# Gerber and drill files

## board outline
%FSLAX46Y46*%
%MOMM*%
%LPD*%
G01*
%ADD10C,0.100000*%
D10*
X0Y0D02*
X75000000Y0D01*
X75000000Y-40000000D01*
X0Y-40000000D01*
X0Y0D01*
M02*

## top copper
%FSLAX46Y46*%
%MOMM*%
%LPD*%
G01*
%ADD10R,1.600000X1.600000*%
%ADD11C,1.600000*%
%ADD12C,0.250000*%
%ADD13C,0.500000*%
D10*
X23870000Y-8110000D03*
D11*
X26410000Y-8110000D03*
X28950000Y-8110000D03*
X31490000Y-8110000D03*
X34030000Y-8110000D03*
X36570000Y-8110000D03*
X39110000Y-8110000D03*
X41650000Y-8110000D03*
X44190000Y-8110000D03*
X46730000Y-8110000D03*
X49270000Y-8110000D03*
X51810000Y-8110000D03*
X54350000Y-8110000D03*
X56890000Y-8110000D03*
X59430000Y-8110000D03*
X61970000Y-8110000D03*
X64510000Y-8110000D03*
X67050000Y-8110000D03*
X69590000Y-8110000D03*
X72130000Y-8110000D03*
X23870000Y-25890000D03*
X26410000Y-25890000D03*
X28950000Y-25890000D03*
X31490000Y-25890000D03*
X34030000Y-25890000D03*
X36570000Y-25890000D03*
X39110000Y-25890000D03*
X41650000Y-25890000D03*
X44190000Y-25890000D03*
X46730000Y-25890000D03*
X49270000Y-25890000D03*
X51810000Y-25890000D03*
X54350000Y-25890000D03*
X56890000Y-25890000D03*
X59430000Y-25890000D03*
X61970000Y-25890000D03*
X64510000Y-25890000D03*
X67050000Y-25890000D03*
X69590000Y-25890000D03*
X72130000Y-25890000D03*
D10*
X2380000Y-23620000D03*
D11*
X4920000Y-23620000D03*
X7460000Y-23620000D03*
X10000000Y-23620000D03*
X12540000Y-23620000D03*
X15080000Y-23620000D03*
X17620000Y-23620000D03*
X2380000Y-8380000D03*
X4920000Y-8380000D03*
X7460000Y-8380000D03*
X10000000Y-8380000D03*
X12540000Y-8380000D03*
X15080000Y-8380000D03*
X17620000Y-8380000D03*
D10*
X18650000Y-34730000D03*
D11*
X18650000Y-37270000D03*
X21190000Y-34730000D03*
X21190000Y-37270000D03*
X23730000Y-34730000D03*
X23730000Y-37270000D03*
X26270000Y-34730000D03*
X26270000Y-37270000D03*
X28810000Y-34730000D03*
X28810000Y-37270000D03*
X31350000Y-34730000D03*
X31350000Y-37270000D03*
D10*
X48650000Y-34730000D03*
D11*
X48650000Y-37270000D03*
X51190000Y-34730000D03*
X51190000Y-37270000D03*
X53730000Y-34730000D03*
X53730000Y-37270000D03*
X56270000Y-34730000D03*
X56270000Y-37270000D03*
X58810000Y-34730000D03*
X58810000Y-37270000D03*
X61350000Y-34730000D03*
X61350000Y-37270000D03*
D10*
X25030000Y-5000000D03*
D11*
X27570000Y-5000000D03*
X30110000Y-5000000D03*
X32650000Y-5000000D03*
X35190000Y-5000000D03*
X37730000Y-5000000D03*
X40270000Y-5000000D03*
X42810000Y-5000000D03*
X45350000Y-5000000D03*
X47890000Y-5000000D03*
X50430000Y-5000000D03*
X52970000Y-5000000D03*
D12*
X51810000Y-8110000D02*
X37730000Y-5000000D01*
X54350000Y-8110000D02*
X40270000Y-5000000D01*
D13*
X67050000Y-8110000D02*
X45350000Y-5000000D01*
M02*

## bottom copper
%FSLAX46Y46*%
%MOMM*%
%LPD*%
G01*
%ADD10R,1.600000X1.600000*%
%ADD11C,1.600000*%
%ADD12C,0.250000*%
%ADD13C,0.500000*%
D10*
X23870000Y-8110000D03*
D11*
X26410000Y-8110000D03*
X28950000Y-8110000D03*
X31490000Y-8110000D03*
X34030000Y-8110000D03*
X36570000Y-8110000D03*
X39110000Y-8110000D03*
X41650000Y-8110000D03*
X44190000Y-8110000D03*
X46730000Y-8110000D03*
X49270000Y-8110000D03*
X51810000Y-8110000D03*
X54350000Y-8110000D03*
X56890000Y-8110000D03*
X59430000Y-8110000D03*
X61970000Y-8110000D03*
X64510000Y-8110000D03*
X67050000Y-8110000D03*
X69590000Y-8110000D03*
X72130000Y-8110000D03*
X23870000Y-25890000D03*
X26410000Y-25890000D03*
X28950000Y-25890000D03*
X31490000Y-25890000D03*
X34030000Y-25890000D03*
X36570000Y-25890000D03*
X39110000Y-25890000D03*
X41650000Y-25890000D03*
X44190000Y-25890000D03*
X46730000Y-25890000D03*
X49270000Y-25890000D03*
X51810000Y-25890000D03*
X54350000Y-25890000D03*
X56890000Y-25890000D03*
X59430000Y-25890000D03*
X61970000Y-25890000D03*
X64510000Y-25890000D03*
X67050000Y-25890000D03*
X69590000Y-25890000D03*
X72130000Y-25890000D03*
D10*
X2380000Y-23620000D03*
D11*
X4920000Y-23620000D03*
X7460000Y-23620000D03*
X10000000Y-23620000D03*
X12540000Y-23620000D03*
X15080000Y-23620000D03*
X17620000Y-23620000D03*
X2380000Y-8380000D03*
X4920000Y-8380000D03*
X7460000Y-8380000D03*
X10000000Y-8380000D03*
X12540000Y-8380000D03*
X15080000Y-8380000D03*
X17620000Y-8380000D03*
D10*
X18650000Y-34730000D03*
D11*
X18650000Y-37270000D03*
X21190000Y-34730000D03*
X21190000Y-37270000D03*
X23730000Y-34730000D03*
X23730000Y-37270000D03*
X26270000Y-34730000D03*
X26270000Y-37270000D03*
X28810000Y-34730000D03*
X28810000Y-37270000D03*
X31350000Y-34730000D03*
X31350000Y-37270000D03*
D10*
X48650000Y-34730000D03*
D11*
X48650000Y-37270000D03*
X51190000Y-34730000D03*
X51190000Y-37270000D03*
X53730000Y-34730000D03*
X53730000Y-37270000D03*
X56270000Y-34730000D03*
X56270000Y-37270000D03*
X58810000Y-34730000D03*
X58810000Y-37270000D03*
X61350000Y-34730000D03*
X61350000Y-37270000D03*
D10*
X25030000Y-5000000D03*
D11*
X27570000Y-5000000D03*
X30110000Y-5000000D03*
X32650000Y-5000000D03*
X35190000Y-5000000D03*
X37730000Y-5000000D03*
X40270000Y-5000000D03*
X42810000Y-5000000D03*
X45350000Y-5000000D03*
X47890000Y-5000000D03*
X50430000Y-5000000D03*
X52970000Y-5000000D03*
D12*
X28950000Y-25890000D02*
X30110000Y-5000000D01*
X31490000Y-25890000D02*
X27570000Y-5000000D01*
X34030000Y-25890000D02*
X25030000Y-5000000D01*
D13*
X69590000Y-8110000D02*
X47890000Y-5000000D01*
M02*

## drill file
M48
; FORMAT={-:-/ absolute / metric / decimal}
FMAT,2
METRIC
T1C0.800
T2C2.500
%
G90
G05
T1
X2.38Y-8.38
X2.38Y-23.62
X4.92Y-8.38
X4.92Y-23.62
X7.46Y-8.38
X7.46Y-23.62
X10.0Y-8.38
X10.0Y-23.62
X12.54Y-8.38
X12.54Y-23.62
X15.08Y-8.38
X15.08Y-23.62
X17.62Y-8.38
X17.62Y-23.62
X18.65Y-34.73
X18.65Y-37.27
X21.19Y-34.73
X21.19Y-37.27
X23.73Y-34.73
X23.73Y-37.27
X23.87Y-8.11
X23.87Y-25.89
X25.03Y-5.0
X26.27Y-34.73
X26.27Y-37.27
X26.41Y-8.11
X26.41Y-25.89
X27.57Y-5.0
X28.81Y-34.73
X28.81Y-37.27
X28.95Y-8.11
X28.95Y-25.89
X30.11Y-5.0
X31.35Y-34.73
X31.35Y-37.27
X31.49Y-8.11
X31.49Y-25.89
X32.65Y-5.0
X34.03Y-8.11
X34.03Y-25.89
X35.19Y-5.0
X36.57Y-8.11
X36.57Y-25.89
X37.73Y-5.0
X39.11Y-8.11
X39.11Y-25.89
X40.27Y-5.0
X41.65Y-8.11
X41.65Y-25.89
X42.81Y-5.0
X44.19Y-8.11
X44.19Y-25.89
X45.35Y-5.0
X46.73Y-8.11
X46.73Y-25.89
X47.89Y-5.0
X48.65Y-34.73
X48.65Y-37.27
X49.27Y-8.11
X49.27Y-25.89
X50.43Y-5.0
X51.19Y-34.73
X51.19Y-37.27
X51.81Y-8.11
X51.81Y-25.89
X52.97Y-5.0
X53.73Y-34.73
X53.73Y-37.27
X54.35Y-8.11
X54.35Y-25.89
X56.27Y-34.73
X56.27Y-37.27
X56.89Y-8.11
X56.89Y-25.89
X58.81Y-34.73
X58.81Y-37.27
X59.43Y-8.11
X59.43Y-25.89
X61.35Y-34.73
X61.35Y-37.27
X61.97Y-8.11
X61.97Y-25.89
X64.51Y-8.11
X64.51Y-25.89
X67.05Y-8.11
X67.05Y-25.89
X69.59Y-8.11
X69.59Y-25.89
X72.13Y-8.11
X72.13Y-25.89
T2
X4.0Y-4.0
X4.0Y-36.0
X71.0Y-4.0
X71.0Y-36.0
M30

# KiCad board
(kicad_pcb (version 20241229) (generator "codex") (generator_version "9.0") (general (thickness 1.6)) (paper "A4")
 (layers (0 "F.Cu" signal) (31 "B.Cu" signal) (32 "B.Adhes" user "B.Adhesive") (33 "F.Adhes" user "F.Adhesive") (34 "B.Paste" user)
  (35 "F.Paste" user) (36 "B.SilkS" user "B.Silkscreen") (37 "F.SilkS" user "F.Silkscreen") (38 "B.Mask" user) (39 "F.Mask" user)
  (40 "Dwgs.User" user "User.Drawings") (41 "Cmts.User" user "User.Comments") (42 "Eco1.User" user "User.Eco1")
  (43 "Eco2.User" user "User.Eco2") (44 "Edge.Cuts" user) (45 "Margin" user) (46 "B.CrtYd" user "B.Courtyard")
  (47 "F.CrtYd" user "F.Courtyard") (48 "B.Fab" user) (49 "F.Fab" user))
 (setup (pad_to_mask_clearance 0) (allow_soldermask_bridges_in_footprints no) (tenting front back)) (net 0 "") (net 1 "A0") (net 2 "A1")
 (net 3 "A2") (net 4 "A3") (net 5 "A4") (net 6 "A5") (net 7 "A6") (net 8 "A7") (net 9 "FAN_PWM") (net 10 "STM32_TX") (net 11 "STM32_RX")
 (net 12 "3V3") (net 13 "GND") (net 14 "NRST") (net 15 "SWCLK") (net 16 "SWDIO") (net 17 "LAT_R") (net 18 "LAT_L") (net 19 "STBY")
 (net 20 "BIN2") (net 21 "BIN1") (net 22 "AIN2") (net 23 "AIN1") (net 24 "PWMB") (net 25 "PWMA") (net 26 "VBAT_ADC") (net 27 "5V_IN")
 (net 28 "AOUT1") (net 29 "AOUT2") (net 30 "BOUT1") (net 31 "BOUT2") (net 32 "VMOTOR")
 (gr_rect (start 0 0) (end 75 40) (stroke (width 0.1) (type solid)) (fill no) (layer "Edge.Cuts"))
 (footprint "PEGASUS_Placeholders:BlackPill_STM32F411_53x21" (layer "F.Cu") (at 48.000 17.000 0)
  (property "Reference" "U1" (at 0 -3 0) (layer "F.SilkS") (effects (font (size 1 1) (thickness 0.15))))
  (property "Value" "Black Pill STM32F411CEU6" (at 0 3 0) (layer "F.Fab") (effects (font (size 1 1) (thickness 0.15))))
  (pad "1" thru_hole rect (at -24.130 -8.890) (size 1.6 1.6) (drill 0.8) (layers "*.Cu" "*.Mask"))
  (pad "2" thru_hole circle (at -21.590 -8.890) (size 1.6 1.6) (drill 0.8) (layers "*.Cu" "*.Mask"))
  (pad "3" thru_hole circle (at -19.050 -8.890) (size 1.6 1.6) (drill 0.8) (layers "*.Cu" "*.Mask") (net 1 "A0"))
  (pad "4" thru_hole circle (at -16.510 -8.890) (size 1.6 1.6) (drill 0.8) (layers "*.Cu" "*.Mask") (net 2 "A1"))
  (pad "5" thru_hole circle (at -13.970 -8.890) (size 1.6 1.6) (drill 0.8) (layers "*.Cu" "*.Mask") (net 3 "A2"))
  (pad "6" thru_hole circle (at -11.430 -8.890) (size 1.6 1.6) (drill 0.8) (layers "*.Cu" "*.Mask") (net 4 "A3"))
  (pad "7" thru_hole circle (at -8.890 -8.890) (size 1.6 1.6) (drill 0.8) (layers "*.Cu" "*.Mask") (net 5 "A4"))
  (pad "8" thru_hole circle (at -6.350 -8.890) (size 1.6 1.6) (drill 0.8) (layers "*.Cu" "*.Mask") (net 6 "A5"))
  (pad "9" thru_hole circle (at -3.810 -8.890) (size 1.6 1.6) (drill 0.8) (layers "*.Cu" "*.Mask") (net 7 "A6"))
  (pad "10" thru_hole circle (at -1.270 -8.890) (size 1.6 1.6) (drill 0.8) (layers "*.Cu" "*.Mask") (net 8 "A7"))
  (pad "11" thru_hole circle (at 1.270 -8.890) (size 1.6 1.6) (drill 0.8) (layers "*.Cu" "*.Mask") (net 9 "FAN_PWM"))
  (pad "12" thru_hole circle (at 3.810 -8.890) (size 1.6 1.6) (drill 0.8) (layers "*.Cu" "*.Mask") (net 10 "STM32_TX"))
  (pad "13" thru_hole circle (at 6.350 -8.890) (size 1.6 1.6) (drill 0.8) (layers "*.Cu" "*.Mask") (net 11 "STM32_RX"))
  (pad "14" thru_hole circle (at 8.890 -8.890) (size 1.6 1.6) (drill 0.8) (layers "*.Cu" "*.Mask"))
  (pad "15" thru_hole circle (at 11.430 -8.890) (size 1.6 1.6) (drill 0.8) (layers "*.Cu" "*.Mask"))
  (pad "16" thru_hole circle (at 13.970 -8.890) (size 1.6 1.6) (drill 0.8) (layers "*.Cu" "*.Mask"))
  (pad "17" thru_hole circle (at 16.510 -8.890) (size 1.6 1.6) (drill 0.8) (layers "*.Cu" "*.Mask"))
  (pad "18" thru_hole circle (at 19.050 -8.890) (size 1.6 1.6) (drill 0.8) (layers "*.Cu" "*.Mask") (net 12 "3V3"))
  (pad "19" thru_hole circle (at 21.590 -8.890) (size 1.6 1.6) (drill 0.8) (layers "*.Cu" "*.Mask") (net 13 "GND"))
  (pad "20" thru_hole circle (at 24.130 -8.890) (size 1.6 1.6) (drill 0.8) (layers "*.Cu" "*.Mask"))
  (pad "40" thru_hole circle (at -24.130 8.890) (size 1.6 1.6) (drill 0.8) (layers "*.Cu" "*.Mask"))
  (pad "39" thru_hole circle (at -21.590 8.890) (size 1.6 1.6) (drill 0.8) (layers "*.Cu" "*.Mask"))
  (pad "38" thru_hole circle (at -19.050 8.890) (size 1.6 1.6) (drill 0.8) (layers "*.Cu" "*.Mask") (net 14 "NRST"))
  (pad "37" thru_hole circle (at -16.510 8.890) (size 1.6 1.6) (drill 0.8) (layers "*.Cu" "*.Mask") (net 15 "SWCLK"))
  (pad "36" thru_hole circle (at -13.970 8.890) (size 1.6 1.6) (drill 0.8) (layers "*.Cu" "*.Mask") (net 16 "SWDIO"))
  (pad "35" thru_hole circle (at -11.430 8.890) (size 1.6 1.6) (drill 0.8) (layers "*.Cu" "*.Mask"))
  (pad "34" thru_hole circle (at -8.890 8.890) (size 1.6 1.6) (drill 0.8) (layers "*.Cu" "*.Mask"))
  (pad "33" thru_hole circle (at -6.350 8.890) (size 1.6 1.6) (drill 0.8) (layers "*.Cu" "*.Mask"))
  (pad "32" thru_hole circle (at -3.810 8.890) (size 1.6 1.6) (drill 0.8) (layers "*.Cu" "*.Mask"))
  (pad "31" thru_hole circle (at -1.270 8.890) (size 1.6 1.6) (drill 0.8) (layers "*.Cu" "*.Mask") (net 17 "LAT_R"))
  (pad "30" thru_hole circle (at 1.270 8.890) (size 1.6 1.6) (drill 0.8) (layers "*.Cu" "*.Mask") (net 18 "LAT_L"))
  (pad "29" thru_hole circle (at 3.810 8.890) (size 1.6 1.6) (drill 0.8) (layers "*.Cu" "*.Mask") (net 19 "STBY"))
  (pad "28" thru_hole circle (at 6.350 8.890) (size 1.6 1.6) (drill 0.8) (layers "*.Cu" "*.Mask") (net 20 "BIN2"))
  (pad "27" thru_hole circle (at 8.890 8.890) (size 1.6 1.6) (drill 0.8) (layers "*.Cu" "*.Mask") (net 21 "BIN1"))
  (pad "26" thru_hole circle (at 11.430 8.890) (size 1.6 1.6) (drill 0.8) (layers "*.Cu" "*.Mask") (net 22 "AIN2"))
  (pad "25" thru_hole circle (at 13.970 8.890) (size 1.6 1.6) (drill 0.8) (layers "*.Cu" "*.Mask") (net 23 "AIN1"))
  (pad "24" thru_hole circle (at 16.510 8.890) (size 1.6 1.6) (drill 0.8) (layers "*.Cu" "*.Mask") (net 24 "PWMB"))
  (pad "23" thru_hole circle (at 19.050 8.890) (size 1.6 1.6) (drill 0.8) (layers "*.Cu" "*.Mask") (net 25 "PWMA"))
  (pad "22" thru_hole circle (at 21.590 8.890) (size 1.6 1.6) (drill 0.8) (layers "*.Cu" "*.Mask") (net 12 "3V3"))
  (pad "21" thru_hole circle (at 24.130 8.890) (size 1.6 1.6) (drill 0.8) (layers "*.Cu" "*.Mask") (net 13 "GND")))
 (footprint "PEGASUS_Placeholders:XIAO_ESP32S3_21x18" (layer "F.Cu") (at 10.000 16.000 90)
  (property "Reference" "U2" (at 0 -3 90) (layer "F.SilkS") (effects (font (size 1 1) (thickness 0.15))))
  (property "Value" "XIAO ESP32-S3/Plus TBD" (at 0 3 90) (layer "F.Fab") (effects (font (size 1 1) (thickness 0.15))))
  (pad "1" thru_hole rect (at -7.620 -7.620) (size 1.6 1.6) (drill 0.8) (layers "*.Cu" "*.Mask"))
  (pad "2" thru_hole circle (at -7.620 -5.080) (size 1.6 1.6) (drill 0.8) (layers "*.Cu" "*.Mask"))
  (pad "3" thru_hole circle (at -7.620 -2.540) (size 1.6 1.6) (drill 0.8) (layers "*.Cu" "*.Mask"))
  (pad "4" thru_hole circle (at -7.620 0.000) (size 1.6 1.6) (drill 0.8) (layers "*.Cu" "*.Mask"))
  (pad "5" thru_hole circle (at -7.620 2.540) (size 1.6 1.6) (drill 0.8) (layers "*.Cu" "*.Mask"))
  (pad "6" thru_hole circle (at -7.620 5.080) (size 1.6 1.6) (drill 0.8) (layers "*.Cu" "*.Mask"))
  (pad "7" thru_hole circle (at -7.620 7.620) (size 1.6 1.6) (drill 0.8) (layers "*.Cu" "*.Mask"))
  (pad "14" thru_hole circle (at 7.620 -7.620) (size 1.6 1.6) (drill 0.8) (layers "*.Cu" "*.Mask"))
  (pad "13" thru_hole circle (at 7.620 -5.080) (size 1.6 1.6) (drill 0.8) (layers "*.Cu" "*.Mask"))
  (pad "12" thru_hole circle (at 7.620 -2.540) (size 1.6 1.6) (drill 0.8) (layers "*.Cu" "*.Mask"))
  (pad "11" thru_hole circle (at 7.620 0.000) (size 1.6 1.6) (drill 0.8) (layers "*.Cu" "*.Mask"))
  (pad "10" thru_hole circle (at 7.620 2.540) (size 1.6 1.6) (drill 0.8) (layers "*.Cu" "*.Mask"))
  (pad "9" thru_hole circle (at 7.620 5.080) (size 1.6 1.6) (drill 0.8) (layers "*.Cu" "*.Mask"))
  (pad "8" thru_hole circle (at 7.620 7.620) (size 1.6 1.6) (drill 0.8) (layers "*.Cu" "*.Mask")))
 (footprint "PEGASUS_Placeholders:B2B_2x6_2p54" (layer "F.Cu") (at 25.000 36.000 0)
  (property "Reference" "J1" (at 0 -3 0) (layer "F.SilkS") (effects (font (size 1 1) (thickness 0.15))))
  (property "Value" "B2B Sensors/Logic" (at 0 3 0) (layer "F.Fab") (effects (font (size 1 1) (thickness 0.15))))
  (pad "1" thru_hole rect (at -6.350 -1.270) (size 1.6 1.6) (drill 0.8) (layers "*.Cu" "*.Mask") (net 12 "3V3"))
  (pad "2" thru_hole circle (at -6.350 1.270) (size 1.6 1.6) (drill 0.8) (layers "*.Cu" "*.Mask") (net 13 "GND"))
  (pad "3" thru_hole circle (at -3.810 -1.270) (size 1.6 1.6) (drill 0.8) (layers "*.Cu" "*.Mask") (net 1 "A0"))
  (pad "4" thru_hole circle (at -3.810 1.270) (size 1.6 1.6) (drill 0.8) (layers "*.Cu" "*.Mask") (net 2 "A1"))
  (pad "5" thru_hole circle (at -1.270 -1.270) (size 1.6 1.6) (drill 0.8) (layers "*.Cu" "*.Mask") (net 3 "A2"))
  (pad "6" thru_hole circle (at -1.270 1.270) (size 1.6 1.6) (drill 0.8) (layers "*.Cu" "*.Mask") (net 4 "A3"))
  (pad "7" thru_hole circle (at 1.270 -1.270) (size 1.6 1.6) (drill 0.8) (layers "*.Cu" "*.Mask") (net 5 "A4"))
  (pad "8" thru_hole circle (at 1.270 1.270) (size 1.6 1.6) (drill 0.8) (layers "*.Cu" "*.Mask") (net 6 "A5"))
  (pad "9" thru_hole circle (at 3.810 -1.270) (size 1.6 1.6) (drill 0.8) (layers "*.Cu" "*.Mask") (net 7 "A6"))
  (pad "10" thru_hole circle (at 3.810 1.270) (size 1.6 1.6) (drill 0.8) (layers "*.Cu" "*.Mask") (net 8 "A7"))
  (pad "11" thru_hole circle (at 6.350 -1.270) (size 1.6 1.6) (drill 0.8) (layers "*.Cu" "*.Mask") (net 18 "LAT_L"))
  (pad "12" thru_hole circle (at 6.350 1.270) (size 1.6 1.6) (drill 0.8) (layers "*.Cu" "*.Mask") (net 17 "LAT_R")))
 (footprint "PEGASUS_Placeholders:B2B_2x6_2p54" (layer "F.Cu") (at 55.000 36.000 0)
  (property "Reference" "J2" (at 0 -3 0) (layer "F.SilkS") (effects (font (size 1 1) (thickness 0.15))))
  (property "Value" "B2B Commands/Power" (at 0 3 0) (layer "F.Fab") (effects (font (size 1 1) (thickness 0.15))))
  (pad "1" thru_hole rect (at -6.350 -1.270) (size 1.6 1.6) (drill 0.8) (layers "*.Cu" "*.Mask") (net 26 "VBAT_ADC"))
  (pad "2" thru_hole circle (at -6.350 1.270) (size 1.6 1.6) (drill 0.8) (layers "*.Cu" "*.Mask") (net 13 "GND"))
  (pad "3" thru_hole circle (at -3.810 -1.270) (size 1.6 1.6) (drill 0.8) (layers "*.Cu" "*.Mask") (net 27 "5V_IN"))
  (pad "4" thru_hole circle (at -3.810 1.270) (size 1.6 1.6) (drill 0.8) (layers "*.Cu" "*.Mask") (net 13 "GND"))
  (pad "5" thru_hole circle (at -1.270 -1.270) (size 1.6 1.6) (drill 0.8) (layers "*.Cu" "*.Mask") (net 25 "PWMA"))
  (pad "6" thru_hole circle (at -1.270 1.270) (size 1.6 1.6) (drill 0.8) (layers "*.Cu" "*.Mask") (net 23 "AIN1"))
  (pad "7" thru_hole circle (at 1.270 -1.270) (size 1.6 1.6) (drill 0.8) (layers "*.Cu" "*.Mask") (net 22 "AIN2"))
  (pad "8" thru_hole circle (at 1.270 1.270) (size 1.6 1.6) (drill 0.8) (layers "*.Cu" "*.Mask") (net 24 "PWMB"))
  (pad "9" thru_hole circle (at 3.810 -1.270) (size 1.6 1.6) (drill 0.8) (layers "*.Cu" "*.Mask") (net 21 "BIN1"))
  (pad "10" thru_hole circle (at 3.810 1.270) (size 1.6 1.6) (drill 0.8) (layers "*.Cu" "*.Mask") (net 20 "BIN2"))
  (pad "11" thru_hole circle (at 6.350 -1.270) (size 1.6 1.6) (drill 0.8) (layers "*.Cu" "*.Mask") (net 19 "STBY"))
  (pad "12" thru_hole circle (at 6.350 1.270) (size 1.6 1.6) (drill 0.8) (layers "*.Cu" "*.Mask") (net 9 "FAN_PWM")))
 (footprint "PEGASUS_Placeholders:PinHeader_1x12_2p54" (layer "F.Cu") (at 39.000 5.000 0)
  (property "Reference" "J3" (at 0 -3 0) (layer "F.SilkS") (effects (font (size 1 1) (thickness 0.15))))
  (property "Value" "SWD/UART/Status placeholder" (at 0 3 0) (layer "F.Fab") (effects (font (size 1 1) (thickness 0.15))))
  (pad "1" thru_hole rect (at -13.970 0.000) (size 1.6 1.6) (drill 0.8) (layers "*.Cu" "*.Mask") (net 16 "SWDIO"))
  (pad "2" thru_hole circle (at -11.430 0.000) (size 1.6 1.6) (drill 0.8) (layers "*.Cu" "*.Mask") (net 15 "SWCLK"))
  (pad "3" thru_hole circle (at -8.890 0.000) (size 1.6 1.6) (drill 0.8) (layers "*.Cu" "*.Mask") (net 14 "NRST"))
  (pad "4" thru_hole circle (at -6.350 0.000) (size 1.6 1.6) (drill 0.8) (layers "*.Cu" "*.Mask") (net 12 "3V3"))
  (pad "5" thru_hole circle (at -3.810 0.000) (size 1.6 1.6) (drill 0.8) (layers "*.Cu" "*.Mask") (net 13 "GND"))
  (pad "6" thru_hole circle (at -1.270 0.000) (size 1.6 1.6) (drill 0.8) (layers "*.Cu" "*.Mask") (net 10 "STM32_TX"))
  (pad "7" thru_hole circle (at 1.270 0.000) (size 1.6 1.6) (drill 0.8) (layers "*.Cu" "*.Mask") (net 11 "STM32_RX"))
  (pad "8" thru_hole circle (at 3.810 0.000) (size 1.6 1.6) (drill 0.8) (layers "*.Cu" "*.Mask") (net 13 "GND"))
  (pad "9" thru_hole circle (at 6.350 0.000) (size 1.6 1.6) (drill 0.8) (layers "*.Cu" "*.Mask") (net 12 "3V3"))
  (pad "10" thru_hole circle (at 8.890 0.000) (size 1.6 1.6) (drill 0.8) (layers "*.Cu" "*.Mask") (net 13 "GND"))
  (pad "11" thru_hole circle (at 11.430 0.000) (size 1.6 1.6) (drill 0.8) (layers "*.Cu" "*.Mask") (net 13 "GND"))
  (pad "12" thru_hole circle (at 13.970 0.000) (size 1.6 1.6) (drill 0.8) (layers "*.Cu" "*.Mask") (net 13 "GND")))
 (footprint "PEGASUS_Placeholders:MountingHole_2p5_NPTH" (layer "F.Cu") (at 4 4)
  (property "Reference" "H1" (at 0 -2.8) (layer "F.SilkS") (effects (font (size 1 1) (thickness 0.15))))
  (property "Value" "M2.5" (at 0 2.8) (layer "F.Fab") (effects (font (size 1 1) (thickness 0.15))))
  (pad "" np_thru_hole circle (at 0 0) (size 2.5 2.5) (drill 2.5) (layers "*.Cu" "*.Mask")))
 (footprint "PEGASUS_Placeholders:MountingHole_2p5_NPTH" (layer "F.Cu") (at 71 4)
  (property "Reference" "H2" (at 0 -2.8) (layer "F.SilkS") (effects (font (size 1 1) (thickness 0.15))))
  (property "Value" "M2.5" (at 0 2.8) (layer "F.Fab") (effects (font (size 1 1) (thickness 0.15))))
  (pad "" np_thru_hole circle (at 0 0) (size 2.5 2.5) (drill 2.5) (layers "*.Cu" "*.Mask")))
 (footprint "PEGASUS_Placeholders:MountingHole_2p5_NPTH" (layer "F.Cu") (at 4 36)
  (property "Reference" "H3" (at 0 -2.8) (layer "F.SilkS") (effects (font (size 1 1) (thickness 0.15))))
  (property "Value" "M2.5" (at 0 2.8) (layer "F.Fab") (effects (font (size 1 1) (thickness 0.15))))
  (pad "" np_thru_hole circle (at 0 0) (size 2.5 2.5) (drill 2.5) (layers "*.Cu" "*.Mask")))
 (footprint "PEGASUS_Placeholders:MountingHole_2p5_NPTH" (layer "F.Cu") (at 71 36)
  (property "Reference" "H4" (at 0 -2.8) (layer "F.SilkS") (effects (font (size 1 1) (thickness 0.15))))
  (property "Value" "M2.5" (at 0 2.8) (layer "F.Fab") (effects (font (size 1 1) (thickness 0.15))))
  (pad "" np_thru_hole circle (at 0 0) (size 2.5 2.5) (drill 2.5) (layers "*.Cu" "*.Mask")))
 (segment (start 51.810 8.110) (end 37.730 5.000) (width 0.25) (layer "F.Cu") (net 10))
 (segment (start 54.350 8.110) (end 40.270 5.000) (width 0.25) (layer "F.Cu") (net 11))
 (segment (start 28.950 25.890) (end 30.110 5.000) (width 0.25) (layer "B.Cu") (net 14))
 (segment (start 31.490 25.890) (end 27.570 5.000) (width 0.25) (layer "B.Cu") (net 15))
 (segment (start 34.030 25.890) (end 25.030 5.000) (width 0.25) (layer "B.Cu") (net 16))
 (segment (start 67.050 8.110) (end 45.350 5.000) (width 0.50) (layer "F.Cu") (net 12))
 (segment (start 69.590 8.110) (end 47.890 5.000) (width 0.50) (layer "B.Cu") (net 13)))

